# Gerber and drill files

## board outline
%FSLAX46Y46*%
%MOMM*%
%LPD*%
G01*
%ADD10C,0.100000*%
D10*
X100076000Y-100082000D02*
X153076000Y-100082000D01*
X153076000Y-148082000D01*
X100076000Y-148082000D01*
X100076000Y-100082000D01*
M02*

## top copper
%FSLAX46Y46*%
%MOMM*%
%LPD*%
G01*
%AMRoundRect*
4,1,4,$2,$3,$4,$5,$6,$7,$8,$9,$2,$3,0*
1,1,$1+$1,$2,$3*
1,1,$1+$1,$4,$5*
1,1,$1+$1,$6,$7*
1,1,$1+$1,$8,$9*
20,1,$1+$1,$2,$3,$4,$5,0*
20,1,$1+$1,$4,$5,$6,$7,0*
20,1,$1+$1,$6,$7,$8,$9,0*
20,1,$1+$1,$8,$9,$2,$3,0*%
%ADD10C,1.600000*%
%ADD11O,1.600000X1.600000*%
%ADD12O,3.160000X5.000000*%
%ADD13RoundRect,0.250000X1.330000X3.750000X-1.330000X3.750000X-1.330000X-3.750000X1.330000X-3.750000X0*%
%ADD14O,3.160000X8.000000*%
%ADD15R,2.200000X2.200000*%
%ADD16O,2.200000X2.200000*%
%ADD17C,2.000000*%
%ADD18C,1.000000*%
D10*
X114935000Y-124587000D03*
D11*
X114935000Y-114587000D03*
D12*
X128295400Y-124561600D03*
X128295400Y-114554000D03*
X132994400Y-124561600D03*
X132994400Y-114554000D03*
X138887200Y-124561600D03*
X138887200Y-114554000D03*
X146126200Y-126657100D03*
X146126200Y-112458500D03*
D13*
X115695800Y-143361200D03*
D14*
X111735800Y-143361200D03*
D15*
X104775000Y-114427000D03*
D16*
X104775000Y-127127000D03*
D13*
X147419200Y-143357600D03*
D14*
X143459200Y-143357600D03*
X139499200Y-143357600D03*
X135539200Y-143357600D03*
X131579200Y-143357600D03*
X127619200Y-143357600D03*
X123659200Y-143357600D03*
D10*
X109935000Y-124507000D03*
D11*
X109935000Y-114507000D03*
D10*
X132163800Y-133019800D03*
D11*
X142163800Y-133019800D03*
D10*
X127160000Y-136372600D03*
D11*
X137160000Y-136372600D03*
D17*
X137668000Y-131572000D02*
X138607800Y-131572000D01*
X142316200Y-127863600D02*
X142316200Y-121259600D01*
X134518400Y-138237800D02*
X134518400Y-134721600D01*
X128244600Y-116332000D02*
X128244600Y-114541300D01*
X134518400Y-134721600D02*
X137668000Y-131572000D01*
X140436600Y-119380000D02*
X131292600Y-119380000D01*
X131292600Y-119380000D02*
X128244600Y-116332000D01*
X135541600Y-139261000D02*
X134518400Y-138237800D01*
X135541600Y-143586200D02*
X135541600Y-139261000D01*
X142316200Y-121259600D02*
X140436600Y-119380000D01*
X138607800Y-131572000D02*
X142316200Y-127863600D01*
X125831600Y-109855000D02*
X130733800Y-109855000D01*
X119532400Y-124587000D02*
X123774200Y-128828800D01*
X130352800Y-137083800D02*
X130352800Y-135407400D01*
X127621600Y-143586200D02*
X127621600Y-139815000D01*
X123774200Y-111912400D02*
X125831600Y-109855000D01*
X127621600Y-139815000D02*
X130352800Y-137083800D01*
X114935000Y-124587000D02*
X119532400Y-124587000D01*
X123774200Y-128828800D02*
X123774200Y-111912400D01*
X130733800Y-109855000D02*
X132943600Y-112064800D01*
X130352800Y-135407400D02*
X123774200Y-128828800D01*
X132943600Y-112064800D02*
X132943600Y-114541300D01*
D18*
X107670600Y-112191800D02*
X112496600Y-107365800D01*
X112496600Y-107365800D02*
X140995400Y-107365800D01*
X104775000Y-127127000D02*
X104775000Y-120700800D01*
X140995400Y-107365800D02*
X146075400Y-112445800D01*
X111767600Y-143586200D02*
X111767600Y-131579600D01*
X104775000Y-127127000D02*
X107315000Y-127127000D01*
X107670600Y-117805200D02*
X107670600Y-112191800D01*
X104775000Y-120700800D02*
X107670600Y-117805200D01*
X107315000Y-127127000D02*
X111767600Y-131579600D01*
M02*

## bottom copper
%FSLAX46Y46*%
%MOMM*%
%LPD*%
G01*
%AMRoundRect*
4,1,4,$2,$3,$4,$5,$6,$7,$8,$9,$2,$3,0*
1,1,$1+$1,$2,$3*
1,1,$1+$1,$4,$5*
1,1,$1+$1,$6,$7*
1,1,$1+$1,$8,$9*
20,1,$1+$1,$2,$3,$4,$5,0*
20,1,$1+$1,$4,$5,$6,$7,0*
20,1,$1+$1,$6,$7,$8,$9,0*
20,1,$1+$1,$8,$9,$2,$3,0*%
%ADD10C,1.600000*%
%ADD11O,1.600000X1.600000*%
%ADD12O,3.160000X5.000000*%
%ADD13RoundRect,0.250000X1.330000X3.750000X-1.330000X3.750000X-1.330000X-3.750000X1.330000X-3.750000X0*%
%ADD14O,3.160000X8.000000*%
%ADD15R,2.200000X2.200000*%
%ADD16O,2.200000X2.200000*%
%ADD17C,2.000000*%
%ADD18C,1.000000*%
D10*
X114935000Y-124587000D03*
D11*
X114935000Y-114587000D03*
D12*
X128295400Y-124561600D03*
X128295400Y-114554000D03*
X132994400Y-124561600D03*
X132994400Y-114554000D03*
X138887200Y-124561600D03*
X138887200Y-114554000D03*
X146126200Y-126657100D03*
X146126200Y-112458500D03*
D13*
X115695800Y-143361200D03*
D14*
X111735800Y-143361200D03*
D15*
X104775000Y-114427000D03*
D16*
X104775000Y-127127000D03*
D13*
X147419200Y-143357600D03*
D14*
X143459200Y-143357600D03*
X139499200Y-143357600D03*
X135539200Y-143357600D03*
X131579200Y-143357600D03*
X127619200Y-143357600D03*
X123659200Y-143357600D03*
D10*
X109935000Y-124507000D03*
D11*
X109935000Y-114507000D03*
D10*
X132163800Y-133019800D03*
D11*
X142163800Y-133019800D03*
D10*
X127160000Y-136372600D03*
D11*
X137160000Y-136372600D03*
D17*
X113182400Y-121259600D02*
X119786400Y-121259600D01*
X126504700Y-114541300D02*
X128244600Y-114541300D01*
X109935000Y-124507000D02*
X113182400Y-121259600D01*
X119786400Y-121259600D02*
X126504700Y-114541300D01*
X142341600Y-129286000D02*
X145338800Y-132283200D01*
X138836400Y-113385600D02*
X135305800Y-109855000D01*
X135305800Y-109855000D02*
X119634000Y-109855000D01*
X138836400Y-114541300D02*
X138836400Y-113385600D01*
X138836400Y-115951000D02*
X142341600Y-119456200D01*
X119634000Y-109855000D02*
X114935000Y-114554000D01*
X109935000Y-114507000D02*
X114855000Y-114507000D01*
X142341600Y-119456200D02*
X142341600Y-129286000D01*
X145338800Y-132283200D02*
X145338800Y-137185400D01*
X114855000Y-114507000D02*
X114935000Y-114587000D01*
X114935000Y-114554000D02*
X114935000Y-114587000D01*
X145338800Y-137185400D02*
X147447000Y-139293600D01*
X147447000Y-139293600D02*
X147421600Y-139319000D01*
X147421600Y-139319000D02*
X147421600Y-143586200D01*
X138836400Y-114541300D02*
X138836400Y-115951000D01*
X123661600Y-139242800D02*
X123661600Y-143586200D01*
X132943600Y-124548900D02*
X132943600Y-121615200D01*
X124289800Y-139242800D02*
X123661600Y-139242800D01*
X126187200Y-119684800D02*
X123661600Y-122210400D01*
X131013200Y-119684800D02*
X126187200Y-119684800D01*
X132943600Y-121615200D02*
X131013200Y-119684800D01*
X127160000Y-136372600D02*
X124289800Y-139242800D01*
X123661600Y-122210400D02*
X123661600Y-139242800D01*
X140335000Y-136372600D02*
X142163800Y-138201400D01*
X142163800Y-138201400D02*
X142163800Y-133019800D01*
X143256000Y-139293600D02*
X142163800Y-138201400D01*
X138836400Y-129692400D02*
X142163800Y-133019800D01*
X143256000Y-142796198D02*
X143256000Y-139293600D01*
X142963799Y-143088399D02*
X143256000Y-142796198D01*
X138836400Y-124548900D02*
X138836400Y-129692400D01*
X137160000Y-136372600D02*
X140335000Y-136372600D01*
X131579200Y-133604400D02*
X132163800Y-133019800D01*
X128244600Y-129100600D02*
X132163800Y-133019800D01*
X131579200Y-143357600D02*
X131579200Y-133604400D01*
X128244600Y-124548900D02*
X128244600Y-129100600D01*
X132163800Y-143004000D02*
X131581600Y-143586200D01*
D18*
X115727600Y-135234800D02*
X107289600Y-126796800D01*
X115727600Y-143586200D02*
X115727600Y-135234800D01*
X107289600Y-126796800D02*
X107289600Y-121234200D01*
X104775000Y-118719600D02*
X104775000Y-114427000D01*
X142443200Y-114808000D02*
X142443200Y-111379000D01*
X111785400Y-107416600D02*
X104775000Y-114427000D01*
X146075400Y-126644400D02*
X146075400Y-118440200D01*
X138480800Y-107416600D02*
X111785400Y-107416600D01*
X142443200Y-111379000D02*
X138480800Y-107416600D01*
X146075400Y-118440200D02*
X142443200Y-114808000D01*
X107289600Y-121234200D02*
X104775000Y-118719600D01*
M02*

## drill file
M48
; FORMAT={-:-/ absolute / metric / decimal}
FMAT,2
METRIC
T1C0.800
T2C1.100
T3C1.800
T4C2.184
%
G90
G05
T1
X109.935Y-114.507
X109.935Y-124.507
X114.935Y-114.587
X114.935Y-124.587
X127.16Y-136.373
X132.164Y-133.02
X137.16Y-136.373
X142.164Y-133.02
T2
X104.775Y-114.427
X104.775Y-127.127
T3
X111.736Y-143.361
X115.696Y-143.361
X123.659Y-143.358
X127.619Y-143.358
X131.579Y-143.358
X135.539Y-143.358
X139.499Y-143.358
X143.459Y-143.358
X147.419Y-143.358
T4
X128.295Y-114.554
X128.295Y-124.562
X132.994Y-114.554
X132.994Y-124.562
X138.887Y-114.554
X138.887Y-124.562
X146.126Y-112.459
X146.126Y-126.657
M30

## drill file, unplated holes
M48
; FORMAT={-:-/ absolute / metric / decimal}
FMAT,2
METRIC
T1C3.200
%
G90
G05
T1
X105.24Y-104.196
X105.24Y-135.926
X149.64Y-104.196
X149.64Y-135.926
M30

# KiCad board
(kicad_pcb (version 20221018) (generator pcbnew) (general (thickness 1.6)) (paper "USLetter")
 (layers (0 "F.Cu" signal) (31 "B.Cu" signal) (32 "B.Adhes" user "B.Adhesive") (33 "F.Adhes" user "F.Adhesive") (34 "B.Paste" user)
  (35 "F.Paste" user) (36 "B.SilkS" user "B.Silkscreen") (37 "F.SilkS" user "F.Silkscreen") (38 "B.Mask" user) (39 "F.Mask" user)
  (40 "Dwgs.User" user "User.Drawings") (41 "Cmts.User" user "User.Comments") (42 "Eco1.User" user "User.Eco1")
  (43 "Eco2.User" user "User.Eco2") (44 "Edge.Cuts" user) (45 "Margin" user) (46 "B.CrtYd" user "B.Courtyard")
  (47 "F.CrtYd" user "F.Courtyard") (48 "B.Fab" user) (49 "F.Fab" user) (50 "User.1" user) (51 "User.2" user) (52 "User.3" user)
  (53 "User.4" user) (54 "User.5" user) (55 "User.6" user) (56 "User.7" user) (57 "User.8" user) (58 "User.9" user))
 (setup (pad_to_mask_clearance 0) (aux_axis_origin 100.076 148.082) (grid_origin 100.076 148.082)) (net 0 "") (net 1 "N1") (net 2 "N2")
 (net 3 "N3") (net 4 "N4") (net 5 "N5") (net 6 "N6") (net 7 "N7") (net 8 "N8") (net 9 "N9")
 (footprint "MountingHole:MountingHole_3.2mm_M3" (layer "F.Cu") (at 149.64 104.196)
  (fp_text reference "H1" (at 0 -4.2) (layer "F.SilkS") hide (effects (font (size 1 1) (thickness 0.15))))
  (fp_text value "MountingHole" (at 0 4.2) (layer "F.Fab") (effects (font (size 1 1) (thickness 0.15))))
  (pad "" np_thru_hole circle (at 0 0) (size 3.2 3.2) (drill 3.2) (layers "*.Cu" "*.Mask")))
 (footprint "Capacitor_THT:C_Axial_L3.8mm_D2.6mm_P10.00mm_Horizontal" (layer "F.Cu") (at 114.935 124.587 90)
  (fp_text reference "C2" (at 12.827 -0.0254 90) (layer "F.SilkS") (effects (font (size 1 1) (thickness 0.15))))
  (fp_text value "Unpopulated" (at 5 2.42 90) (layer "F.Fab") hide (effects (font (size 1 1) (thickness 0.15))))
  (pad "1" thru_hole circle (at 0 0 90) (size 1.6 1.6) (drill 0.8) (layers "*.Cu" "*.Mask") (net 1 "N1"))
  (pad "2" thru_hole oval (at 10 0 90) (size 1.6 1.6) (drill 0.8) (layers "*.Cu" "*.Mask") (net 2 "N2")))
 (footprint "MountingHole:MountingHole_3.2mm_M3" (layer "F.Cu") (at 149.64 135.926)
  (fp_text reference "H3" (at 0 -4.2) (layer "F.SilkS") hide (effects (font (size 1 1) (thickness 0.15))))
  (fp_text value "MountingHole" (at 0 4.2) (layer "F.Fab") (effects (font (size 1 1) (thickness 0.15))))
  (pad "" np_thru_hole circle (at 0 0) (size 3.2 3.2) (drill 3.2) (layers "*.Cu" "*.Mask")))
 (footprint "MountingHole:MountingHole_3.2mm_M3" (layer "F.Cu") (at 105.24 104.196)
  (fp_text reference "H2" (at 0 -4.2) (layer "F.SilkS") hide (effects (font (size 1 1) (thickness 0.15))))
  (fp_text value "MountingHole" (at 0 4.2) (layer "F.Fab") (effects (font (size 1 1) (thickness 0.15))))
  (pad "" np_thru_hole circle (at 0 0) (size 3.2 3.2) (drill 3.2) (layers "*.Cu" "*.Mask")))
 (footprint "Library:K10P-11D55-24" (layer "F.Cu") (at 128.2954 124.5616 90)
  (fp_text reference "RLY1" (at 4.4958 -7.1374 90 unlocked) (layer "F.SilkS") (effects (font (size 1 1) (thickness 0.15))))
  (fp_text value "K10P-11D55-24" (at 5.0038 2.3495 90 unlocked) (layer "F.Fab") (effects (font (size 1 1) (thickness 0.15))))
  (pad "1" thru_hole oval (at 0 0 90) (size 5 3.16) (drill 2.1844) (layers "*.Cu" "*.Mask") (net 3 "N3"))
  (pad "2" thru_hole oval (at 10.0076 0 90) (size 5 3.16) (drill 2.1844) (layers "*.Cu" "*.Mask") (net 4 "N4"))
  (pad "3" thru_hole oval (at 0 4.699 90) (size 5 3.16) (drill 2.1844) (layers "*.Cu" "*.Mask") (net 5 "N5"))
  (pad "4" thru_hole oval (at 10.0076 4.699 90) (size 5 3.16) (drill 2.1844) (layers "*.Cu" "*.Mask") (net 1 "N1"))
  (pad "5" thru_hole oval (at 0 10.5918 90) (size 5 3.16) (drill 2.1844) (layers "*.Cu" "*.Mask") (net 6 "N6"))
  (pad "6" thru_hole oval (at 10.0076 10.5918 90) (size 5 3.16) (drill 2.1844) (layers "*.Cu" "*.Mask") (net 2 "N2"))
  (pad "7" thru_hole oval (at -2.0955 17.8308 90) (size 5 3.16) (drill 2.1844) (layers "*.Cu" "*.Mask") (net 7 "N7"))
  (pad "8" thru_hole oval (at 12.1031 17.8308 90) (size 5 3.16) (drill 2.1844) (layers "*.Cu" "*.Mask") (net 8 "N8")))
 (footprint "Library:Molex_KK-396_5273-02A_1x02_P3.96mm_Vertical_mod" (layer "F.Cu") (at 115.6958 143.3612 180)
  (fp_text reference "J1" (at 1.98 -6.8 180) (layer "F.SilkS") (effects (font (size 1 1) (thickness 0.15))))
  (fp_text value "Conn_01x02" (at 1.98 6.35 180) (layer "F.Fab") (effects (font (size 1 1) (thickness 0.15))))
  (pad "1" thru_hole roundrect (at 0 0 180) (size 3.16 8) (drill 1.8) (layers "*.Cu" "*.Mask") (roundrect_rratio 0.07911392405) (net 7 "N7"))
  (pad "2" thru_hole oval (at 3.96 0 180) (size 3.16 8) (drill 1.8) (layers "*.Cu" "*.Mask") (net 8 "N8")))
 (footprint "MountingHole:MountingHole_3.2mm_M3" (layer "F.Cu") (at 105.24 135.926)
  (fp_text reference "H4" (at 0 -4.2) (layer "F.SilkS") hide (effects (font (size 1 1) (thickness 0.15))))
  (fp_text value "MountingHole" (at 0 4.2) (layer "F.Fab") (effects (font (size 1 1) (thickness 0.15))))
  (pad "" np_thru_hole circle (at 0 0) (size 3.2 3.2) (drill 3.2) (layers "*.Cu" "*.Mask")))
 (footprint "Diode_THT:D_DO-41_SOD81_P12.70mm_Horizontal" (layer "F.Cu") (at 104.775 114.427 -90)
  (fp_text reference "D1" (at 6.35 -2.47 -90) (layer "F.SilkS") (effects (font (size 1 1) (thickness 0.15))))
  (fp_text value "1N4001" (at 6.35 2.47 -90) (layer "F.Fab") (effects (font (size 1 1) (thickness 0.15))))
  (pad "1" thru_hole rect (at 0 0 270) (size 2.2 2.2) (drill 1.1) (layers "*.Cu" "*.Mask") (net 7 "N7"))
  (pad "2" thru_hole oval (at 12.7 0 270) (size 2.2 2.2) (drill 1.1) (layers "*.Cu" "*.Mask") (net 8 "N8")))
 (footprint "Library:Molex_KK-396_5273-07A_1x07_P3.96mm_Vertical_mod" (layer "F.Cu") (at 147.4192 143.3576 180)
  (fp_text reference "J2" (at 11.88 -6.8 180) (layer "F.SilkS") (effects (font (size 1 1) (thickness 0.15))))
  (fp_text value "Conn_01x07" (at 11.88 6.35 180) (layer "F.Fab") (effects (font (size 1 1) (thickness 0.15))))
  (pad "1" thru_hole roundrect (at 0 0 180) (size 3.16 8) (drill 1.8) (layers "*.Cu" "*.Mask") (roundrect_rratio 0.07911392405) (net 2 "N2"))
  (pad "2" thru_hole oval (at 3.96 0 180) (size 3.16 8) (drill 1.8) (layers "*.Cu" "*.Mask") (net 6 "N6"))
  (pad "3" thru_hole oval (at 7.92 0 180) (size 3.16 8) (drill 1.8) (layers "*.Cu" "*.Mask") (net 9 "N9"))
  (pad "4" thru_hole oval (at 11.88 0 180) (size 3.16 8) (drill 1.8) (layers "*.Cu" "*.Mask") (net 4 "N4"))
  (pad "5" thru_hole oval (at 15.84 0 180) (size 3.16 8) (drill 1.8) (layers "*.Cu" "*.Mask") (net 3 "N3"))
  (pad "6" thru_hole oval (at 19.8 0 180) (size 3.16 8) (drill 1.8) (layers "*.Cu" "*.Mask") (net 1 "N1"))
  (pad "7" thru_hole oval (at 23.76 0 180) (size 3.16 8) (drill 1.8) (layers "*.Cu" "*.Mask") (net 5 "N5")))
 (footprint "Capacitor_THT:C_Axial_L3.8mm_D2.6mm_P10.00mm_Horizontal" (layer "F.Cu") (at 109.935 124.507 90)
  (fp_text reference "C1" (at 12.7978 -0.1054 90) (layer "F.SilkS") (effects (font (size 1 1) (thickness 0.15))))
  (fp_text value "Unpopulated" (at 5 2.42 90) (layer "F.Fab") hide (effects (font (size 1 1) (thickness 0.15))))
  (pad "1" thru_hole circle (at 0 0 90) (size 1.6 1.6) (drill 0.8) (layers "*.Cu" "*.Mask") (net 4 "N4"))
  (pad "2" thru_hole oval (at 10 0 90) (size 1.6 1.6) (drill 0.8) (layers "*.Cu" "*.Mask") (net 2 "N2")))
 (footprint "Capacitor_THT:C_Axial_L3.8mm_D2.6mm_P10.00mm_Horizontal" (layer "F.Cu") (at 132.1638 133.0198)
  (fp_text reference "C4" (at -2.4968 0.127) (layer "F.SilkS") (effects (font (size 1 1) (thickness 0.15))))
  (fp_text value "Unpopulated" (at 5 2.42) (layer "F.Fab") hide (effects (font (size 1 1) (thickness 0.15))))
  (pad "1" thru_hole circle (at 0 0) (size 1.6 1.6) (drill 0.8) (layers "*.Cu" "*.Mask") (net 3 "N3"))
  (pad "2" thru_hole oval (at 10 0) (size 1.6 1.6) (drill 0.8) (layers "*.Cu" "*.Mask") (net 6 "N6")))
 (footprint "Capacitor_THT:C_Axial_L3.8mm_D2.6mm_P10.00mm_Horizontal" (layer "F.Cu") (at 127.16 136.3726)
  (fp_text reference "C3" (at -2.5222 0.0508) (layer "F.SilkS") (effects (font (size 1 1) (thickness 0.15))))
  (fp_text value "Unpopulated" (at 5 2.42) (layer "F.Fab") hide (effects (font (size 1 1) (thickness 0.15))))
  (pad "1" thru_hole circle (at 0 0) (size 1.6 1.6) (drill 0.8) (layers "*.Cu" "*.Mask") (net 5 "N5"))
  (pad "2" thru_hole oval (at 10 0) (size 1.6 1.6) (drill 0.8) (layers "*.Cu" "*.Mask") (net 6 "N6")))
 (gr_rect locked (start 100.076 100.082) (end 153.076 148.082) (stroke (width 0.1) (type default)) (fill none) (layer "Edge.Cuts"))
 (segment (start 137.668 131.572) (end 138.6078 131.572) (width 2) (layer "F.Cu") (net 4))
 (segment (start 142.3162 127.8636) (end 142.3162 121.2596) (width 2) (layer "F.Cu") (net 4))
 (segment (start 134.5184 138.2378) (end 134.5184 134.7216) (width 2) (layer "F.Cu") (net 4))
 (segment (start 128.2446 116.332) (end 128.2446 114.5413) (width 2) (layer "F.Cu") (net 4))
 (segment (start 134.5184 134.7216) (end 137.668 131.572) (width 2) (layer "F.Cu") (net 4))
 (segment (start 140.4366 119.38) (end 131.2926 119.38) (width 2) (layer "F.Cu") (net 4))
 (segment (start 131.2926 119.38) (end 128.2446 116.332) (width 2) (layer "F.Cu") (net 4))
 (segment (start 135.5416 139.261) (end 134.5184 138.2378) (width 2) (layer "F.Cu") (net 4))
 (segment (start 135.5416 143.5862) (end 135.5416 139.261) (width 2) (layer "F.Cu") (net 4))
 (segment (start 142.3162 121.2596) (end 140.4366 119.38) (width 2) (layer "F.Cu") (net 4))
 (segment (start 138.6078 131.572) (end 142.3162 127.8636) (width 2) (layer "F.Cu") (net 4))
 (segment (start 113.1824 121.2596) (end 119.7864 121.2596) (width 2) (layer "B.Cu") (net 4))
 (segment (start 126.5047 114.5413) (end 128.2446 114.5413) (width 2) (layer "B.Cu") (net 4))
 (segment (start 109.935 124.507) (end 113.1824 121.2596) (width 2) (layer "B.Cu") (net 4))
 (segment (start 119.7864 121.2596) (end 126.5047 114.5413) (width 2) (layer "B.Cu") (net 4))
 (segment (start 142.3416 129.286) (end 145.3388 132.2832) (width 2) (layer "B.Cu") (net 2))
 (segment (start 138.8364 113.3856) (end 135.3058 109.855) (width 2) (layer "B.Cu") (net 2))
 (segment (start 135.3058 109.855) (end 119.634 109.855) (width 2) (layer "B.Cu") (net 2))
 (segment (start 138.8364 114.5413) (end 138.8364 113.3856) (width 2) (layer "B.Cu") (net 2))
 (segment (start 138.8364 115.951) (end 142.3416 119.4562) (width 2) (layer "B.Cu") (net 2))
 (segment (start 119.634 109.855) (end 114.935 114.554) (width 2) (layer "B.Cu") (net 2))
 (segment (start 109.935 114.507) (end 114.855 114.507) (width 2) (layer "B.Cu") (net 2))
 (segment (start 142.3416 119.4562) (end 142.3416 129.286) (width 2) (layer "B.Cu") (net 2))
 (segment (start 145.3388 132.2832) (end 145.3388 137.1854) (width 2) (layer "B.Cu") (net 2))
 (segment (start 114.855 114.507) (end 114.935 114.587) (width 2) (layer "B.Cu") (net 2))
 (segment (start 114.935 114.554) (end 114.935 114.587) (width 2) (layer "B.Cu") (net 2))
 (segment (start 145.3388 137.1854) (end 147.447 139.2936) (width 2) (layer "B.Cu") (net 2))
 (segment (start 147.447 139.2936) (end 147.4216 139.319) (width 2) (layer "B.Cu") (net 2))
 (segment (start 147.4216 139.319) (end 147.4216 143.5862) (width 2) (layer "B.Cu") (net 2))
 (segment (start 138.8364 114.5413) (end 138.8364 115.951) (width 2) (layer "B.Cu") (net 2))
 (segment (start 125.8316 109.855) (end 130.7338 109.855) (width 2) (layer "F.Cu") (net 1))
 (segment (start 119.5324 124.587) (end 123.7742 128.8288) (width 2) (layer "F.Cu") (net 1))
 (segment (start 130.3528 137.0838) (end 130.3528 135.4074) (width 2) (layer "F.Cu") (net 1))
 (segment (start 127.6216 143.5862) (end 127.6216 139.815) (width 2) (layer "F.Cu") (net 1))
 (segment (start 123.7742 111.9124) (end 125.8316 109.855) (width 2) (layer "F.Cu") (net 1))
 (segment (start 127.6216 139.815) (end 130.3528 137.0838) (width 2) (layer "F.Cu") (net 1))
 (segment (start 114.935 124.587) (end 119.5324 124.587) (width 2) (layer "F.Cu") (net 1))
 (segment (start 123.7742 128.8288) (end 123.7742 111.9124) (width 2) (layer "F.Cu") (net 1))
 (segment (start 130.7338 109.855) (end 132.9436 112.0648) (width 2) (layer "F.Cu") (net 1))
 (segment (start 130.3528 135.4074) (end 123.7742 128.8288) (width 2) (layer "F.Cu") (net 1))
 (segment (start 132.9436 112.0648) (end 132.9436 114.5413) (width 2) (layer "F.Cu") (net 1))
 (segment (start 123.6616 139.2428) (end 123.6616 143.5862) (width 2) (layer "B.Cu") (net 5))
 (segment (start 132.9436 124.5489) (end 132.9436 121.6152) (width 2) (layer "B.Cu") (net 5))
 (segment (start 124.2898 139.2428) (end 123.6616 139.2428) (width 2) (layer "B.Cu") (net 5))
 (segment (start 126.1872 119.6848) (end 123.6616 122.2104) (width 2) (layer "B.Cu") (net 5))
 (segment (start 131.0132 119.6848) (end 126.1872 119.6848) (width 2) (layer "B.Cu") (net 5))
 (segment (start 132.9436 121.6152) (end 131.0132 119.6848) (width 2) (layer "B.Cu") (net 5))
 (segment (start 127.16 136.3726) (end 124.2898 139.2428) (width 2) (layer "B.Cu") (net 5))
 (segment (start 123.6616 122.2104) (end 123.6616 139.2428) (width 2) (layer "B.Cu") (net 5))
 (segment (start 140.335 136.3726) (end 142.1638 138.2014) (width 2) (layer "B.Cu") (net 6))
 (segment (start 142.1638 138.2014) (end 142.1638 133.0198) (width 2) (layer "B.Cu") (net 6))
 (segment (start 143.256 139.2936) (end 142.1638 138.2014) (width 2) (layer "B.Cu") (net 6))
 (segment (start 138.8364 129.6924) (end 142.1638 133.0198) (width 2) (layer "B.Cu") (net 6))
 (segment (start 143.256 142.796198) (end 143.256 139.2936) (width 2) (layer "B.Cu") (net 6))
 (segment (start 142.963799 143.088399) (end 143.256 142.796198) (width 2) (layer "B.Cu") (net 6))
 (segment (start 138.8364 124.5489) (end 138.8364 129.6924) (width 2) (layer "B.Cu") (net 6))
 (segment (start 137.16 136.3726) (end 140.335 136.3726) (width 2) (layer "B.Cu") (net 6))
 (segment (start 131.5792 133.6044) (end 132.1638 133.0198) (width 2) (layer "B.Cu") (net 3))
 (segment (start 128.2446 129.1006) (end 132.1638 133.0198) (width 2) (layer "B.Cu") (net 3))
 (segment (start 131.5792 143.3576) (end 131.5792 133.6044) (width 2) (layer "B.Cu") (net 3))
 (segment (start 128.2446 124.5489) (end 128.2446 129.1006) (width 2) (layer "B.Cu") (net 3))
 (segment (start 132.1638 143.004) (end 131.5816 143.5862) (width 2) (layer "B.Cu") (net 3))
 (segment (start 115.7276 135.2348) (end 107.2896 126.7968) (width 1) (layer "B.Cu") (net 7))
 (segment (start 115.7276 143.5862) (end 115.7276 135.2348) (width 1) (layer "B.Cu") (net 7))
 (segment (start 107.2896 126.7968) (end 107.2896 121.2342) (width 1) (layer "B.Cu") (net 7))
 (segment (start 104.775 118.7196) (end 104.775 114.427) (width 1) (layer "B.Cu") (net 7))
 (segment (start 142.4432 114.808) (end 142.4432 111.379) (width 1) (layer "B.Cu") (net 7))
 (segment (start 111.7854 107.4166) (end 104.775 114.427) (width 1) (layer "B.Cu") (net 7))
 (segment (start 146.0754 126.6444) (end 146.0754 118.4402) (width 1) (layer "B.Cu") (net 7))
 (segment (start 138.4808 107.4166) (end 111.7854 107.4166) (width 1) (layer "B.Cu") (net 7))
 (segment (start 142.4432 111.379) (end 138.4808 107.4166) (width 1) (layer "B.Cu") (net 7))
 (segment (start 146.0754 118.4402) (end 142.4432 114.808) (width 1) (layer "B.Cu") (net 7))
 (segment (start 107.2896 121.2342) (end 104.775 118.7196) (width 1) (layer "B.Cu") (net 7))
 (segment (start 107.6706 112.1918) (end 112.4966 107.3658) (width 1) (layer "F.Cu") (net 8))
 (segment (start 112.4966 107.3658) (end 140.9954 107.3658) (width 1) (layer "F.Cu") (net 8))
 (segment (start 104.775 127.127) (end 104.775 120.7008) (width 1) (layer "F.Cu") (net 8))
 (segment (start 140.9954 107.3658) (end 146.0754 112.4458) (width 1) (layer "F.Cu") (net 8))
 (segment (start 111.7676 143.5862) (end 111.7676 131.5796) (width 1) (layer "F.Cu") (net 8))
 (segment (start 104.775 127.127) (end 107.315 127.127) (width 1) (layer "F.Cu") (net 8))
 (segment (start 107.6706 117.8052) (end 107.6706 112.1918) (width 1) (layer "F.Cu") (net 8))
 (segment (start 104.775 120.7008) (end 107.6706 117.8052) (width 1) (layer "F.Cu") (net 8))
 (segment (start 107.315 127.127) (end 111.7676 131.5796) (width 1) (layer "F.Cu") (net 8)))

